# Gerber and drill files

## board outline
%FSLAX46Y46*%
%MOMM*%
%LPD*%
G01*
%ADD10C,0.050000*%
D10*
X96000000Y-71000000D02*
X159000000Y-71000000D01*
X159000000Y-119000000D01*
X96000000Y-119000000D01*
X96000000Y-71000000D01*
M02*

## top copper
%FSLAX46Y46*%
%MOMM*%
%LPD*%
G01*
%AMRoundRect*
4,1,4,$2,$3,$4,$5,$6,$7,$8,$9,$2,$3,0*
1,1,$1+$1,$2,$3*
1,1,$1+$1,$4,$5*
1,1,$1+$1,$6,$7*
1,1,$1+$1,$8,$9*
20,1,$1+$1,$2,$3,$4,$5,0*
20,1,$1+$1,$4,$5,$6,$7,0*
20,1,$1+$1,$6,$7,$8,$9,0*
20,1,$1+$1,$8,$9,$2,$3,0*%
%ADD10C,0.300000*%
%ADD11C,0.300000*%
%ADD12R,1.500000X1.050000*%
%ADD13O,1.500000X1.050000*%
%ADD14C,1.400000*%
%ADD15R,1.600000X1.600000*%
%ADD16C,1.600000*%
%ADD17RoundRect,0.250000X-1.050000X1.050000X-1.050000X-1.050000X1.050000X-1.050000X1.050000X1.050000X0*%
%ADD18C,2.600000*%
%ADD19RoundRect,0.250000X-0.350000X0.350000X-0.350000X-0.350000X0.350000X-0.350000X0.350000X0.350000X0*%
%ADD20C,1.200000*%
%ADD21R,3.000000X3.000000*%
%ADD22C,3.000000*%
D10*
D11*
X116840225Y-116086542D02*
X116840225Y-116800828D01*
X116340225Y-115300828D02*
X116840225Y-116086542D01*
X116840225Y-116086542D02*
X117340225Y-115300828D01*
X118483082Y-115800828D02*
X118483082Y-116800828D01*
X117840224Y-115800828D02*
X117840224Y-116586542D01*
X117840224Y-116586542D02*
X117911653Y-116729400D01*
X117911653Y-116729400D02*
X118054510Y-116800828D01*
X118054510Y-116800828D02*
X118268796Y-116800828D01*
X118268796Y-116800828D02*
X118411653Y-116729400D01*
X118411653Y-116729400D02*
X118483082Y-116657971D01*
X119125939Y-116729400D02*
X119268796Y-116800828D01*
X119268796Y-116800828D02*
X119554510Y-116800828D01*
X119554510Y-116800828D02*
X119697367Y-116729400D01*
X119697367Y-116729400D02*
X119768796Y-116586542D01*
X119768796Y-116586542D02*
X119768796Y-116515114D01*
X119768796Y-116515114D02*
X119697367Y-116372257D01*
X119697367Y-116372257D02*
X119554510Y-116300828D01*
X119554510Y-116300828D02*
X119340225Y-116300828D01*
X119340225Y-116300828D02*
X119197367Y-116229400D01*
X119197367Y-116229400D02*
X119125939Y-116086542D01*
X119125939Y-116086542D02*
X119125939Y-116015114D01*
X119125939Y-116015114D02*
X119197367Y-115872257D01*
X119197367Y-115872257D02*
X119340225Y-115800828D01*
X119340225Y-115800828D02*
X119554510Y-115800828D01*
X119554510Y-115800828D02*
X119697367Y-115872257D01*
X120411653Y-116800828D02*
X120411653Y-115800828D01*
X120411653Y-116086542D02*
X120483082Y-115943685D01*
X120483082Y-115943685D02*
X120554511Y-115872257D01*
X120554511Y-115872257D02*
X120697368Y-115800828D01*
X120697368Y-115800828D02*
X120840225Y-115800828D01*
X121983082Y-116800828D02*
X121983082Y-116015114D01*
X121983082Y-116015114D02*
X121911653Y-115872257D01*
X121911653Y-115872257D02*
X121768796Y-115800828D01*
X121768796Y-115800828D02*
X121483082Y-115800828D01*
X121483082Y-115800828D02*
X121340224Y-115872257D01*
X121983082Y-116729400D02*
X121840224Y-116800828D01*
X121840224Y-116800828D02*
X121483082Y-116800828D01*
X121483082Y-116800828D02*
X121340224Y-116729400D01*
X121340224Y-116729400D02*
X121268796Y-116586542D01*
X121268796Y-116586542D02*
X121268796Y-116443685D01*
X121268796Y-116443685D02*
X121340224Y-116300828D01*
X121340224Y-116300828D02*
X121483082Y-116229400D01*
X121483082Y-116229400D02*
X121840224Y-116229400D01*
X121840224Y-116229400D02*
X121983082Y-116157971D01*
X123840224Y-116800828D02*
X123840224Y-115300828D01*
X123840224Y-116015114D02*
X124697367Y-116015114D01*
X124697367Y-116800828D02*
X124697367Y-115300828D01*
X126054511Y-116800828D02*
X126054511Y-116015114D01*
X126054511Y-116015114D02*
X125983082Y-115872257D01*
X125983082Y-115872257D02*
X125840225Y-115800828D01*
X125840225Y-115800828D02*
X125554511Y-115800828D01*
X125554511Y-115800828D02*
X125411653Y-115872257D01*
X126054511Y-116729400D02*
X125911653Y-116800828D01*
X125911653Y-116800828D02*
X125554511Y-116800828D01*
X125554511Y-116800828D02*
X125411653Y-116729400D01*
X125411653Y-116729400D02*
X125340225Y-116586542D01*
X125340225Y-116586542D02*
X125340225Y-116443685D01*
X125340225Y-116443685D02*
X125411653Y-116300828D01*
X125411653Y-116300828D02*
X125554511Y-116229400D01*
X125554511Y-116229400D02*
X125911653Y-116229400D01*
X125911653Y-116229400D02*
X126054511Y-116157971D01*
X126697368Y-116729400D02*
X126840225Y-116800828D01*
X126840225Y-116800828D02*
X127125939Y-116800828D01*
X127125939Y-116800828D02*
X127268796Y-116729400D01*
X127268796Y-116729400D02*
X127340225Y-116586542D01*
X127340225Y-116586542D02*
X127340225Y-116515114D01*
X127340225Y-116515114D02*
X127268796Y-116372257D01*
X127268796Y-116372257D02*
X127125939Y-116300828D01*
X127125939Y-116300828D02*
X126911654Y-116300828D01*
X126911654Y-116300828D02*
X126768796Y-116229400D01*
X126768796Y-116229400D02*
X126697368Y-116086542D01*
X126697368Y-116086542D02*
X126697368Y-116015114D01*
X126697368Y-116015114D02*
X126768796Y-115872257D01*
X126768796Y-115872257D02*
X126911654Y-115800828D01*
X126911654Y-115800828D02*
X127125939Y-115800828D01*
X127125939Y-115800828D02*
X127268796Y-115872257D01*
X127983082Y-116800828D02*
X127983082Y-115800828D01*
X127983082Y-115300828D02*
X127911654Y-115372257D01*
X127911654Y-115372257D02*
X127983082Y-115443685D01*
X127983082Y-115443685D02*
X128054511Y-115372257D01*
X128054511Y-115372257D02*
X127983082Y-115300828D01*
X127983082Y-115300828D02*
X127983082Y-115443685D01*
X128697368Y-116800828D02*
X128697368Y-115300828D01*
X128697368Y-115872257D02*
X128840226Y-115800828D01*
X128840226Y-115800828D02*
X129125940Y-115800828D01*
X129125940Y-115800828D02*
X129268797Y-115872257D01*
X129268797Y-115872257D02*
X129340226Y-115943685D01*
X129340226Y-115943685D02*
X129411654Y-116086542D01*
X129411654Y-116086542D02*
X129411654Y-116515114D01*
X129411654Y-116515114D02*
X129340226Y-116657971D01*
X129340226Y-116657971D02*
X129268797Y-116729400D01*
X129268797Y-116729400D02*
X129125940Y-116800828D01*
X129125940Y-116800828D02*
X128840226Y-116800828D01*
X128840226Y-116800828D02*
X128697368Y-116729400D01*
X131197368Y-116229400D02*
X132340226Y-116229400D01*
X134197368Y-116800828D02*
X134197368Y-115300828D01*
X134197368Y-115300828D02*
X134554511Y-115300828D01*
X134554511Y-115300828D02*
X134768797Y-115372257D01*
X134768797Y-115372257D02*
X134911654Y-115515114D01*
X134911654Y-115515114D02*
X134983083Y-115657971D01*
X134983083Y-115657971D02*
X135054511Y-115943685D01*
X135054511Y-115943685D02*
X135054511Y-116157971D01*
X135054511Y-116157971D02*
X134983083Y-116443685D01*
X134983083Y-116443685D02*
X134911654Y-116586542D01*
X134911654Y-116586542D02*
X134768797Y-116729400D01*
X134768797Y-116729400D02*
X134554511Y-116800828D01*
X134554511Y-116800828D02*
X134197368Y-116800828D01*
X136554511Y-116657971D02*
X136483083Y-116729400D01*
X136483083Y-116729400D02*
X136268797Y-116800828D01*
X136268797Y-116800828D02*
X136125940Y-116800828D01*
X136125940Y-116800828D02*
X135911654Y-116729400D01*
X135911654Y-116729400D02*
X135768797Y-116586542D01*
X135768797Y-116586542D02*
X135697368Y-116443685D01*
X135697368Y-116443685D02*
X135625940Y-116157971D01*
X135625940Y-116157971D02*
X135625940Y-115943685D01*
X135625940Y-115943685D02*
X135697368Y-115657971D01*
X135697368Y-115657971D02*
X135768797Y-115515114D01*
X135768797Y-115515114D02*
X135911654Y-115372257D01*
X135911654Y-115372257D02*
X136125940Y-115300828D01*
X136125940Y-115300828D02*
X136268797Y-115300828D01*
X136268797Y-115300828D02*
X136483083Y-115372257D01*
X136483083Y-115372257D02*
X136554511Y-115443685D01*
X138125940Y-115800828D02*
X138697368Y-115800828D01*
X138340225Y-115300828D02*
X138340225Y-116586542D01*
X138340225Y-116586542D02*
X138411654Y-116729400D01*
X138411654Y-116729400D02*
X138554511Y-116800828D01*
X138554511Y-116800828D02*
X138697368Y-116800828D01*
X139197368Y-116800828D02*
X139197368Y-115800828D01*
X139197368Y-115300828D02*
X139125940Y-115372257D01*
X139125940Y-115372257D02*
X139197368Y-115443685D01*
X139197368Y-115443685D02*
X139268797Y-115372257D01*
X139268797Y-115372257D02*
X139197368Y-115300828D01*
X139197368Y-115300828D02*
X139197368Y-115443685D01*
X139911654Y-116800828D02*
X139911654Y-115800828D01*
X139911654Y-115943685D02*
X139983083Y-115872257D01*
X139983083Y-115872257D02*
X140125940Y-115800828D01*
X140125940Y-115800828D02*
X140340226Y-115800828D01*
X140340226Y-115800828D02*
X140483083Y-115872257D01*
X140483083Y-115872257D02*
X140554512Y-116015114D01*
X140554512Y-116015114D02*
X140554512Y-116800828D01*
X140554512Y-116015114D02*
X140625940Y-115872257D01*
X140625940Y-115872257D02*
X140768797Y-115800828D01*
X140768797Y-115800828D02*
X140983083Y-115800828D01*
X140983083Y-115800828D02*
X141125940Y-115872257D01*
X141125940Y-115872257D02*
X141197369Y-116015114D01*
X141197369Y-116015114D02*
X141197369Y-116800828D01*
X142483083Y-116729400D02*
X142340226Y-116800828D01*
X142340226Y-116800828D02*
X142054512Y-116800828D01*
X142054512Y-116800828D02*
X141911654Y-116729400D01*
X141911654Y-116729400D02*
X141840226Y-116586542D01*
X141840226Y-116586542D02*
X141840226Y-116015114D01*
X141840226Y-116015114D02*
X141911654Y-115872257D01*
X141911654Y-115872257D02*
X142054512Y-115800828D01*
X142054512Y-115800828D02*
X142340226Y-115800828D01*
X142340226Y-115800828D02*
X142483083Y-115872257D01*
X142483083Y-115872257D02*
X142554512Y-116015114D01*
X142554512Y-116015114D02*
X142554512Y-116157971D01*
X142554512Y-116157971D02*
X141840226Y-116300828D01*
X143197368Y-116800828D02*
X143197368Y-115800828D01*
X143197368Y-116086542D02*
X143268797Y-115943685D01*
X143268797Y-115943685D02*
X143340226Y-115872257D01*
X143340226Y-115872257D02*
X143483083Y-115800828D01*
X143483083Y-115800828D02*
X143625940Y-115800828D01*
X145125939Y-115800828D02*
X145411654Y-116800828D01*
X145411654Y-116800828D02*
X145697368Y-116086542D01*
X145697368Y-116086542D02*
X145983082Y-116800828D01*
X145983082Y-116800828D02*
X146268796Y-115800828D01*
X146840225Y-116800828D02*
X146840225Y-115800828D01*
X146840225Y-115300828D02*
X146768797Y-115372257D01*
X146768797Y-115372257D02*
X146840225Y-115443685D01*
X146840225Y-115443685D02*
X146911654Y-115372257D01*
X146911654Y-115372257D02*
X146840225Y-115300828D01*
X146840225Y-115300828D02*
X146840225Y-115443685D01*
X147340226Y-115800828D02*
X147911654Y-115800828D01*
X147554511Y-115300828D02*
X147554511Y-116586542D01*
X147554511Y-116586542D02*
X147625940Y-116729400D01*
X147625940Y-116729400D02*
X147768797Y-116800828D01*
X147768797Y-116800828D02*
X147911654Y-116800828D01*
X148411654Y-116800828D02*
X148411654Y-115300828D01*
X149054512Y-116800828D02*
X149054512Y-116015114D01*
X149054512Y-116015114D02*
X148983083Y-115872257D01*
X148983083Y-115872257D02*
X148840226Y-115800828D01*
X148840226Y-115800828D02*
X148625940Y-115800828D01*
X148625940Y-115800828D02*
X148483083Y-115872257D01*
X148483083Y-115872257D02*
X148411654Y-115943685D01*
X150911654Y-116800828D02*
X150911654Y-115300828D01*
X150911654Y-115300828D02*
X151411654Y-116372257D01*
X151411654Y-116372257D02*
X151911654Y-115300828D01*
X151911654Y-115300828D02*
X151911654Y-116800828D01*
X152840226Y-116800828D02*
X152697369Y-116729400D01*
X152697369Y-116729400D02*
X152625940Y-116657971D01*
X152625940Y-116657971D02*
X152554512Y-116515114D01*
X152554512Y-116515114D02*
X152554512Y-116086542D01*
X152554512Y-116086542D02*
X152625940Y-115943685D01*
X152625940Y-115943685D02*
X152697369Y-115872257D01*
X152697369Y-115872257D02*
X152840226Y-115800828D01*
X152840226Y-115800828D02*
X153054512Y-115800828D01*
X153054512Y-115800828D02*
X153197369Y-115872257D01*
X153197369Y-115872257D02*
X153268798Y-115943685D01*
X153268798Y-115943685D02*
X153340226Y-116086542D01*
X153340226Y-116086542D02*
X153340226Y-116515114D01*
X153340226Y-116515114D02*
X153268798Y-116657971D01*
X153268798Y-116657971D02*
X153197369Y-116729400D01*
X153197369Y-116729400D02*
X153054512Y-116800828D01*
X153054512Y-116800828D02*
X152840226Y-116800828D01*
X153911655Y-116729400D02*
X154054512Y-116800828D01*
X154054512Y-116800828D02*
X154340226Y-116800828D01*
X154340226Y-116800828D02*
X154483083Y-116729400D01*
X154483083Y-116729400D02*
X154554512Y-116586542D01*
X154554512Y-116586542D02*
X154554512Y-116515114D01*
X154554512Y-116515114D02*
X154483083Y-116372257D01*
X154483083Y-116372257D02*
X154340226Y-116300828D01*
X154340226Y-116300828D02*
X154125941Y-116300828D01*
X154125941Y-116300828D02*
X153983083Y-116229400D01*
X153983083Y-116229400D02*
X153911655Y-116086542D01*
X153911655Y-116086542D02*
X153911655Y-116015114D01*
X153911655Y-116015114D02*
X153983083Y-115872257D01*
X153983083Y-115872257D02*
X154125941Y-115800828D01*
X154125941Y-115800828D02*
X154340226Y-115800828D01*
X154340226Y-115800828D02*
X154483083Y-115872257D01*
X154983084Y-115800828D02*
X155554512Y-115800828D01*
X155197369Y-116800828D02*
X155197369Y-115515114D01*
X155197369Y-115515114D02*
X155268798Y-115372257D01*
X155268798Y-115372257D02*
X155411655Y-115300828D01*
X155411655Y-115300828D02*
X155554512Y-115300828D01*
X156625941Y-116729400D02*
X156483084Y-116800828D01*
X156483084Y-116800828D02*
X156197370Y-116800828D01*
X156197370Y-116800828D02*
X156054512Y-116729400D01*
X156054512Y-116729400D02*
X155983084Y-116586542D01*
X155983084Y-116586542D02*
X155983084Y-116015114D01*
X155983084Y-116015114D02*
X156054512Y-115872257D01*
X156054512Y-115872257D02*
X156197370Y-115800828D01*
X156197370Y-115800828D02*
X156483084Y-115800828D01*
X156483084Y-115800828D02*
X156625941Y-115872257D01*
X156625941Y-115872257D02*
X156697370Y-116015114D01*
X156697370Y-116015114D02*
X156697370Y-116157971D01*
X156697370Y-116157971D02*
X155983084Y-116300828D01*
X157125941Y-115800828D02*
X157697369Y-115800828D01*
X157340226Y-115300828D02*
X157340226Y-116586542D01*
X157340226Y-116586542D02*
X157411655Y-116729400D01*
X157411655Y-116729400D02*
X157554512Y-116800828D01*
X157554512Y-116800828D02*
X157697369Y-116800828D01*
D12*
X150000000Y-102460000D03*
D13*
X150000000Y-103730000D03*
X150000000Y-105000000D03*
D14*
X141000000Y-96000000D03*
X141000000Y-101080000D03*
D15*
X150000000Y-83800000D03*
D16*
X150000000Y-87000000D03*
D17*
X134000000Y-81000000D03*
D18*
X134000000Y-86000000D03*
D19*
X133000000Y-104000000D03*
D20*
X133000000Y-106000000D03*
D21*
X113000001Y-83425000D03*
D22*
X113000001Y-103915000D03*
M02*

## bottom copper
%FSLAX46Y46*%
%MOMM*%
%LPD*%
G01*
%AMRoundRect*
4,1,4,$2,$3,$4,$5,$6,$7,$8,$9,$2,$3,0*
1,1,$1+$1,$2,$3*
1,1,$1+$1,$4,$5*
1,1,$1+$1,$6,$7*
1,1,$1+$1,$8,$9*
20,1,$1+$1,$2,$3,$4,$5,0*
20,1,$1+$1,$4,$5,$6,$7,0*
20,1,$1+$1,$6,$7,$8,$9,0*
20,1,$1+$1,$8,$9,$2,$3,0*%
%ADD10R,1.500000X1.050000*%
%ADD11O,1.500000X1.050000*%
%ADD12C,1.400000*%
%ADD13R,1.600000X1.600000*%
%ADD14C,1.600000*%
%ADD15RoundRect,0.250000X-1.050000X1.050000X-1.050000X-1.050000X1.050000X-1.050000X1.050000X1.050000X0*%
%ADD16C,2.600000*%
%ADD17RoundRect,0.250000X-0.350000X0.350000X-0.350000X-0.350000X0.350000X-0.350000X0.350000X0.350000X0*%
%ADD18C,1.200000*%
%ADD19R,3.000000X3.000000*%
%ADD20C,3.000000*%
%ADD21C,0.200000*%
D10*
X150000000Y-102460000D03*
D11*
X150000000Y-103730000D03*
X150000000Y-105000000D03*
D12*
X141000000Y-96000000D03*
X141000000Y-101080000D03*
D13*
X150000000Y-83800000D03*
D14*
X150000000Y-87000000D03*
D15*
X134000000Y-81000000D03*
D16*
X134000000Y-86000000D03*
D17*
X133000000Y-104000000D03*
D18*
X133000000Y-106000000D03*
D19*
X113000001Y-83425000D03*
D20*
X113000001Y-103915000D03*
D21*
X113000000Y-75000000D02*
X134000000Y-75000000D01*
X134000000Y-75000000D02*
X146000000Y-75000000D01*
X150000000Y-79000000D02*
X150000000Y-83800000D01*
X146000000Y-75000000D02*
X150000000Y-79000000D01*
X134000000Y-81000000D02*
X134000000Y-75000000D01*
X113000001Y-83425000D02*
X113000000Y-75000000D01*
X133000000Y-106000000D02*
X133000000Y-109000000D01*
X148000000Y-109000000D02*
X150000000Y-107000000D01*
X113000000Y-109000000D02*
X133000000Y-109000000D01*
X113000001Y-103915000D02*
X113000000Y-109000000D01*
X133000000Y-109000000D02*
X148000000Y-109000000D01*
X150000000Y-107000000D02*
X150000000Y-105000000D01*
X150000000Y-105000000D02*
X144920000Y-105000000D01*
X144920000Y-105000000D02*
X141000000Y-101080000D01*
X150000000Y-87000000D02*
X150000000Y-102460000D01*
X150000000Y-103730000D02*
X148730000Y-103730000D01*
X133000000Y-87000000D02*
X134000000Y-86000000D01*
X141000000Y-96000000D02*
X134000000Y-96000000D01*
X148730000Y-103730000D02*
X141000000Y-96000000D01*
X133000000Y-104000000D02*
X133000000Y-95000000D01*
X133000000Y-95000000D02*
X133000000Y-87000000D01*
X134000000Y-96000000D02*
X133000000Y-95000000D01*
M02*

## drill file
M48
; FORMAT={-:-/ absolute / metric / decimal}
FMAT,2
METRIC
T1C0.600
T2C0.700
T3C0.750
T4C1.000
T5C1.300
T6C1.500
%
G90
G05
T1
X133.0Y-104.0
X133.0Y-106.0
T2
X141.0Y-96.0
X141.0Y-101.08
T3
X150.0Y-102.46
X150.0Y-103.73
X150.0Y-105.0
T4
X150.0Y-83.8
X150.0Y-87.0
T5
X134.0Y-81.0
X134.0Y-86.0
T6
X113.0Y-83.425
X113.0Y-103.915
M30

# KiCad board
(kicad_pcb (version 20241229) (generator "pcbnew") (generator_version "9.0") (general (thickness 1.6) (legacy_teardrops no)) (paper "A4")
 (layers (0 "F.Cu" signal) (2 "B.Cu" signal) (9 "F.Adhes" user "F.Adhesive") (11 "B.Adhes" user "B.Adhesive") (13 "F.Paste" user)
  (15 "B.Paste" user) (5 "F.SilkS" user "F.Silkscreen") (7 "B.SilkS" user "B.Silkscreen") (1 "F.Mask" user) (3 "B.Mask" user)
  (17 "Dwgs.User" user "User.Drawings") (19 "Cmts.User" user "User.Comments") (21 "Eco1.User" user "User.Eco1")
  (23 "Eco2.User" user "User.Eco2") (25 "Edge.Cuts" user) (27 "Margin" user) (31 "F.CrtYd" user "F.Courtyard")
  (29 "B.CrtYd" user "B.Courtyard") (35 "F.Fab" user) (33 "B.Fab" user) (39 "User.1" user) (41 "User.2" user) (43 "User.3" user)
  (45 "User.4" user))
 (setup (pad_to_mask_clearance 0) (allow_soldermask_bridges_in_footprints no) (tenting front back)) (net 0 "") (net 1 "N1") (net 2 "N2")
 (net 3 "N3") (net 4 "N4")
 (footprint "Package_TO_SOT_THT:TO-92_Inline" (layer "F.Cu") (at 150 102.46 -90)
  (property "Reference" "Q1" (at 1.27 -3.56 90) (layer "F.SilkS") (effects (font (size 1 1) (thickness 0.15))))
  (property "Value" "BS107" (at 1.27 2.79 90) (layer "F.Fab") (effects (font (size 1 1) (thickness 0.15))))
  (pad "1" thru_hole rect (at 0 0 270) (size 1.05 1.5) (drill 0.75) (layers "*.Cu" "*.Mask") (remove_unused_layers no) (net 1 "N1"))
  (pad "2" thru_hole oval (at 1.27 0 270) (size 1.05 1.5) (drill 0.75) (layers "*.Cu" "*.Mask") (remove_unused_layers no) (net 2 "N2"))
  (pad "3" thru_hole oval (at 2.54 0 270) (size 1.05 1.5) (drill 0.75) (layers "*.Cu" "*.Mask") (remove_unused_layers no) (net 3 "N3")))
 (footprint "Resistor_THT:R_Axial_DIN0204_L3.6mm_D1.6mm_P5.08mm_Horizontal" (layer "F.Cu") (at 141 96 -90)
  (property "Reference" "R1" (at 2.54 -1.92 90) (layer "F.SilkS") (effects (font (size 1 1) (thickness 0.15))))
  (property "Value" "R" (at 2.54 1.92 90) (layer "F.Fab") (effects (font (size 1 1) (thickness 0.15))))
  (pad "1" thru_hole circle (at 0 0 270) (size 1.4 1.4) (drill 0.7) (layers "*.Cu" "*.Mask") (remove_unused_layers no) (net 2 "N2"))
  (pad "2" thru_hole circle (at 5.08 0 270) (size 1.4 1.4) (drill 0.7) (layers "*.Cu" "*.Mask") (remove_unused_layers no) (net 3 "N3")))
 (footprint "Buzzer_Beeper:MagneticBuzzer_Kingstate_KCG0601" (layer "F.Cu") (at 150 83.8 -90)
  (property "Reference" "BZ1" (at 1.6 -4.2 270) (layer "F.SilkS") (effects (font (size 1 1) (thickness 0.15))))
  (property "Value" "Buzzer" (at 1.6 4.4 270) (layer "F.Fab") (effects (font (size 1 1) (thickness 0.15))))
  (pad "1" thru_hole rect (at 0 0 270) (size 1.6 1.6) (drill 1) (layers "*.Cu" "*.Mask") (remove_unused_layers no) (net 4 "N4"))
  (pad "2" thru_hole circle (at 3.2 0 270) (size 1.6 1.6) (drill 1) (layers "*.Cu" "*.Mask") (remove_unused_layers no) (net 1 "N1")))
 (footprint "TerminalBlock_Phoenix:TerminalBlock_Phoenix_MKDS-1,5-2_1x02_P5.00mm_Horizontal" (layer "F.Cu") (at 134 81 -90)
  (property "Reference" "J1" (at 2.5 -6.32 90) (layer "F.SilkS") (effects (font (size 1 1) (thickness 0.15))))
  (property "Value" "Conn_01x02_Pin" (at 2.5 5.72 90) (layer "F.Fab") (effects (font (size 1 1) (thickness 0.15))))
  (pad "1" thru_hole roundrect (at 0 0 270) (size 2.6 2.6) (drill 1.3) (layers "*.Cu" "*.Mask") (remove_unused_layers no)
   (roundrect_rratio 0.096154) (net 4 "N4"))
  (pad "2" thru_hole circle (at 5 0 270) (size 2.6 2.6) (drill 1.3) (layers "*.Cu" "*.Mask") (remove_unused_layers no) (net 2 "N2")))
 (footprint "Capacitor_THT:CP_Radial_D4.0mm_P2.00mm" (layer "F.Cu") (at 133 104 -90)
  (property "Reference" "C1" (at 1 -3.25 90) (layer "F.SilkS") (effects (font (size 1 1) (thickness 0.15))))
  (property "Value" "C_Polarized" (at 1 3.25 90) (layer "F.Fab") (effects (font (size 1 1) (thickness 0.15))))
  (pad "1" thru_hole roundrect (at 0 0 270) (size 1.2 1.2) (drill 0.6) (layers "*.Cu" "*.Mask") (remove_unused_layers no)
   (roundrect_rratio 0.208333) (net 2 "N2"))
  (pad "2" thru_hole circle (at 2 0 270) (size 1.2 1.2) (drill 0.6) (layers "*.Cu" "*.Mask") (remove_unused_layers no) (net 3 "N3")))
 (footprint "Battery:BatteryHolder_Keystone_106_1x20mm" (layer "F.Cu") (at 113.000001 83.425 -90)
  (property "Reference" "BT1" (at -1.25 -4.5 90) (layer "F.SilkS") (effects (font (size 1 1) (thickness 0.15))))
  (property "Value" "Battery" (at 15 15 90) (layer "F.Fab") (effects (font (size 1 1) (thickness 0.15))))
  (pad "1" thru_hole rect (at 0 0 270) (size 3 3) (drill 1.5) (layers "*.Cu" "*.Mask") (remove_unused_layers no) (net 4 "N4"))
  (pad "2" thru_hole circle (at 20.49 0 270) (size 3 3) (drill 1.5) (layers "*.Cu" "*.Mask") (remove_unused_layers no) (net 3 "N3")))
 (gr_poly (pts (xy 96 71) (xy 159 71) (xy 159 119) (xy 96 119)) (stroke (width 0.05) (type solid)) (fill no) (layer "Edge.Cuts"))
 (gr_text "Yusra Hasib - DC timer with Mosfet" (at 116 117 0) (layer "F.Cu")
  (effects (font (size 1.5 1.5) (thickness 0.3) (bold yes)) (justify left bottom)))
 (segment (start 113 75) (end 134 75) (width 0.2) (layer "B.Cu") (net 4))
 (segment (start 134 75) (end 146 75) (width 0.2) (layer "B.Cu") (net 4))
 (segment (start 150 79) (end 150 83.8) (width 0.2) (layer "B.Cu") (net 4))
 (segment (start 146 75) (end 150 79) (width 0.2) (layer "B.Cu") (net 4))
 (segment (start 134 81) (end 134 75) (width 0.2) (layer "B.Cu") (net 4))
 (segment (start 113.000001 83.425) (end 113 75) (width 0.2) (layer "B.Cu") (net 4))
 (segment (start 133 106) (end 133 109) (width 0.2) (layer "B.Cu") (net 3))
 (segment (start 148 109) (end 150 107) (width 0.2) (layer "B.Cu") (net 3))
 (segment (start 113 109) (end 133 109) (width 0.2) (layer "B.Cu") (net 3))
 (segment (start 113.000001 103.915) (end 113 109) (width 0.2) (layer "B.Cu") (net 3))
 (segment (start 133 109) (end 148 109) (width 0.2) (layer "B.Cu") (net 3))
 (segment (start 150 107) (end 150 105) (width 0.2) (layer "B.Cu") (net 3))
 (segment (start 150 105) (end 144.92 105) (width 0.2) (layer "B.Cu") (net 3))
 (segment (start 144.92 105) (end 141 101.08) (width 0.2) (layer "B.Cu") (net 3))
 (segment (start 150 87) (end 150 102.46) (width 0.2) (layer "B.Cu") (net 1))
 (segment (start 150 103.73) (end 148.73 103.73) (width 0.2) (layer "B.Cu") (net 2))
 (segment (start 133 87) (end 134 86) (width 0.2) (layer "B.Cu") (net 2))
 (segment (start 141 96) (end 134 96) (width 0.2) (layer "B.Cu") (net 2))
 (segment (start 148.73 103.73) (end 141 96) (width 0.2) (layer "B.Cu") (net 2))
 (segment (start 133 104) (end 133 95) (width 0.2) (layer "B.Cu") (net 2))
 (segment (start 133 95) (end 133 87) (width 0.2) (layer "B.Cu") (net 2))
 (segment (start 134 96) (end 133 95) (width 0.2) (layer "B.Cu") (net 2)))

